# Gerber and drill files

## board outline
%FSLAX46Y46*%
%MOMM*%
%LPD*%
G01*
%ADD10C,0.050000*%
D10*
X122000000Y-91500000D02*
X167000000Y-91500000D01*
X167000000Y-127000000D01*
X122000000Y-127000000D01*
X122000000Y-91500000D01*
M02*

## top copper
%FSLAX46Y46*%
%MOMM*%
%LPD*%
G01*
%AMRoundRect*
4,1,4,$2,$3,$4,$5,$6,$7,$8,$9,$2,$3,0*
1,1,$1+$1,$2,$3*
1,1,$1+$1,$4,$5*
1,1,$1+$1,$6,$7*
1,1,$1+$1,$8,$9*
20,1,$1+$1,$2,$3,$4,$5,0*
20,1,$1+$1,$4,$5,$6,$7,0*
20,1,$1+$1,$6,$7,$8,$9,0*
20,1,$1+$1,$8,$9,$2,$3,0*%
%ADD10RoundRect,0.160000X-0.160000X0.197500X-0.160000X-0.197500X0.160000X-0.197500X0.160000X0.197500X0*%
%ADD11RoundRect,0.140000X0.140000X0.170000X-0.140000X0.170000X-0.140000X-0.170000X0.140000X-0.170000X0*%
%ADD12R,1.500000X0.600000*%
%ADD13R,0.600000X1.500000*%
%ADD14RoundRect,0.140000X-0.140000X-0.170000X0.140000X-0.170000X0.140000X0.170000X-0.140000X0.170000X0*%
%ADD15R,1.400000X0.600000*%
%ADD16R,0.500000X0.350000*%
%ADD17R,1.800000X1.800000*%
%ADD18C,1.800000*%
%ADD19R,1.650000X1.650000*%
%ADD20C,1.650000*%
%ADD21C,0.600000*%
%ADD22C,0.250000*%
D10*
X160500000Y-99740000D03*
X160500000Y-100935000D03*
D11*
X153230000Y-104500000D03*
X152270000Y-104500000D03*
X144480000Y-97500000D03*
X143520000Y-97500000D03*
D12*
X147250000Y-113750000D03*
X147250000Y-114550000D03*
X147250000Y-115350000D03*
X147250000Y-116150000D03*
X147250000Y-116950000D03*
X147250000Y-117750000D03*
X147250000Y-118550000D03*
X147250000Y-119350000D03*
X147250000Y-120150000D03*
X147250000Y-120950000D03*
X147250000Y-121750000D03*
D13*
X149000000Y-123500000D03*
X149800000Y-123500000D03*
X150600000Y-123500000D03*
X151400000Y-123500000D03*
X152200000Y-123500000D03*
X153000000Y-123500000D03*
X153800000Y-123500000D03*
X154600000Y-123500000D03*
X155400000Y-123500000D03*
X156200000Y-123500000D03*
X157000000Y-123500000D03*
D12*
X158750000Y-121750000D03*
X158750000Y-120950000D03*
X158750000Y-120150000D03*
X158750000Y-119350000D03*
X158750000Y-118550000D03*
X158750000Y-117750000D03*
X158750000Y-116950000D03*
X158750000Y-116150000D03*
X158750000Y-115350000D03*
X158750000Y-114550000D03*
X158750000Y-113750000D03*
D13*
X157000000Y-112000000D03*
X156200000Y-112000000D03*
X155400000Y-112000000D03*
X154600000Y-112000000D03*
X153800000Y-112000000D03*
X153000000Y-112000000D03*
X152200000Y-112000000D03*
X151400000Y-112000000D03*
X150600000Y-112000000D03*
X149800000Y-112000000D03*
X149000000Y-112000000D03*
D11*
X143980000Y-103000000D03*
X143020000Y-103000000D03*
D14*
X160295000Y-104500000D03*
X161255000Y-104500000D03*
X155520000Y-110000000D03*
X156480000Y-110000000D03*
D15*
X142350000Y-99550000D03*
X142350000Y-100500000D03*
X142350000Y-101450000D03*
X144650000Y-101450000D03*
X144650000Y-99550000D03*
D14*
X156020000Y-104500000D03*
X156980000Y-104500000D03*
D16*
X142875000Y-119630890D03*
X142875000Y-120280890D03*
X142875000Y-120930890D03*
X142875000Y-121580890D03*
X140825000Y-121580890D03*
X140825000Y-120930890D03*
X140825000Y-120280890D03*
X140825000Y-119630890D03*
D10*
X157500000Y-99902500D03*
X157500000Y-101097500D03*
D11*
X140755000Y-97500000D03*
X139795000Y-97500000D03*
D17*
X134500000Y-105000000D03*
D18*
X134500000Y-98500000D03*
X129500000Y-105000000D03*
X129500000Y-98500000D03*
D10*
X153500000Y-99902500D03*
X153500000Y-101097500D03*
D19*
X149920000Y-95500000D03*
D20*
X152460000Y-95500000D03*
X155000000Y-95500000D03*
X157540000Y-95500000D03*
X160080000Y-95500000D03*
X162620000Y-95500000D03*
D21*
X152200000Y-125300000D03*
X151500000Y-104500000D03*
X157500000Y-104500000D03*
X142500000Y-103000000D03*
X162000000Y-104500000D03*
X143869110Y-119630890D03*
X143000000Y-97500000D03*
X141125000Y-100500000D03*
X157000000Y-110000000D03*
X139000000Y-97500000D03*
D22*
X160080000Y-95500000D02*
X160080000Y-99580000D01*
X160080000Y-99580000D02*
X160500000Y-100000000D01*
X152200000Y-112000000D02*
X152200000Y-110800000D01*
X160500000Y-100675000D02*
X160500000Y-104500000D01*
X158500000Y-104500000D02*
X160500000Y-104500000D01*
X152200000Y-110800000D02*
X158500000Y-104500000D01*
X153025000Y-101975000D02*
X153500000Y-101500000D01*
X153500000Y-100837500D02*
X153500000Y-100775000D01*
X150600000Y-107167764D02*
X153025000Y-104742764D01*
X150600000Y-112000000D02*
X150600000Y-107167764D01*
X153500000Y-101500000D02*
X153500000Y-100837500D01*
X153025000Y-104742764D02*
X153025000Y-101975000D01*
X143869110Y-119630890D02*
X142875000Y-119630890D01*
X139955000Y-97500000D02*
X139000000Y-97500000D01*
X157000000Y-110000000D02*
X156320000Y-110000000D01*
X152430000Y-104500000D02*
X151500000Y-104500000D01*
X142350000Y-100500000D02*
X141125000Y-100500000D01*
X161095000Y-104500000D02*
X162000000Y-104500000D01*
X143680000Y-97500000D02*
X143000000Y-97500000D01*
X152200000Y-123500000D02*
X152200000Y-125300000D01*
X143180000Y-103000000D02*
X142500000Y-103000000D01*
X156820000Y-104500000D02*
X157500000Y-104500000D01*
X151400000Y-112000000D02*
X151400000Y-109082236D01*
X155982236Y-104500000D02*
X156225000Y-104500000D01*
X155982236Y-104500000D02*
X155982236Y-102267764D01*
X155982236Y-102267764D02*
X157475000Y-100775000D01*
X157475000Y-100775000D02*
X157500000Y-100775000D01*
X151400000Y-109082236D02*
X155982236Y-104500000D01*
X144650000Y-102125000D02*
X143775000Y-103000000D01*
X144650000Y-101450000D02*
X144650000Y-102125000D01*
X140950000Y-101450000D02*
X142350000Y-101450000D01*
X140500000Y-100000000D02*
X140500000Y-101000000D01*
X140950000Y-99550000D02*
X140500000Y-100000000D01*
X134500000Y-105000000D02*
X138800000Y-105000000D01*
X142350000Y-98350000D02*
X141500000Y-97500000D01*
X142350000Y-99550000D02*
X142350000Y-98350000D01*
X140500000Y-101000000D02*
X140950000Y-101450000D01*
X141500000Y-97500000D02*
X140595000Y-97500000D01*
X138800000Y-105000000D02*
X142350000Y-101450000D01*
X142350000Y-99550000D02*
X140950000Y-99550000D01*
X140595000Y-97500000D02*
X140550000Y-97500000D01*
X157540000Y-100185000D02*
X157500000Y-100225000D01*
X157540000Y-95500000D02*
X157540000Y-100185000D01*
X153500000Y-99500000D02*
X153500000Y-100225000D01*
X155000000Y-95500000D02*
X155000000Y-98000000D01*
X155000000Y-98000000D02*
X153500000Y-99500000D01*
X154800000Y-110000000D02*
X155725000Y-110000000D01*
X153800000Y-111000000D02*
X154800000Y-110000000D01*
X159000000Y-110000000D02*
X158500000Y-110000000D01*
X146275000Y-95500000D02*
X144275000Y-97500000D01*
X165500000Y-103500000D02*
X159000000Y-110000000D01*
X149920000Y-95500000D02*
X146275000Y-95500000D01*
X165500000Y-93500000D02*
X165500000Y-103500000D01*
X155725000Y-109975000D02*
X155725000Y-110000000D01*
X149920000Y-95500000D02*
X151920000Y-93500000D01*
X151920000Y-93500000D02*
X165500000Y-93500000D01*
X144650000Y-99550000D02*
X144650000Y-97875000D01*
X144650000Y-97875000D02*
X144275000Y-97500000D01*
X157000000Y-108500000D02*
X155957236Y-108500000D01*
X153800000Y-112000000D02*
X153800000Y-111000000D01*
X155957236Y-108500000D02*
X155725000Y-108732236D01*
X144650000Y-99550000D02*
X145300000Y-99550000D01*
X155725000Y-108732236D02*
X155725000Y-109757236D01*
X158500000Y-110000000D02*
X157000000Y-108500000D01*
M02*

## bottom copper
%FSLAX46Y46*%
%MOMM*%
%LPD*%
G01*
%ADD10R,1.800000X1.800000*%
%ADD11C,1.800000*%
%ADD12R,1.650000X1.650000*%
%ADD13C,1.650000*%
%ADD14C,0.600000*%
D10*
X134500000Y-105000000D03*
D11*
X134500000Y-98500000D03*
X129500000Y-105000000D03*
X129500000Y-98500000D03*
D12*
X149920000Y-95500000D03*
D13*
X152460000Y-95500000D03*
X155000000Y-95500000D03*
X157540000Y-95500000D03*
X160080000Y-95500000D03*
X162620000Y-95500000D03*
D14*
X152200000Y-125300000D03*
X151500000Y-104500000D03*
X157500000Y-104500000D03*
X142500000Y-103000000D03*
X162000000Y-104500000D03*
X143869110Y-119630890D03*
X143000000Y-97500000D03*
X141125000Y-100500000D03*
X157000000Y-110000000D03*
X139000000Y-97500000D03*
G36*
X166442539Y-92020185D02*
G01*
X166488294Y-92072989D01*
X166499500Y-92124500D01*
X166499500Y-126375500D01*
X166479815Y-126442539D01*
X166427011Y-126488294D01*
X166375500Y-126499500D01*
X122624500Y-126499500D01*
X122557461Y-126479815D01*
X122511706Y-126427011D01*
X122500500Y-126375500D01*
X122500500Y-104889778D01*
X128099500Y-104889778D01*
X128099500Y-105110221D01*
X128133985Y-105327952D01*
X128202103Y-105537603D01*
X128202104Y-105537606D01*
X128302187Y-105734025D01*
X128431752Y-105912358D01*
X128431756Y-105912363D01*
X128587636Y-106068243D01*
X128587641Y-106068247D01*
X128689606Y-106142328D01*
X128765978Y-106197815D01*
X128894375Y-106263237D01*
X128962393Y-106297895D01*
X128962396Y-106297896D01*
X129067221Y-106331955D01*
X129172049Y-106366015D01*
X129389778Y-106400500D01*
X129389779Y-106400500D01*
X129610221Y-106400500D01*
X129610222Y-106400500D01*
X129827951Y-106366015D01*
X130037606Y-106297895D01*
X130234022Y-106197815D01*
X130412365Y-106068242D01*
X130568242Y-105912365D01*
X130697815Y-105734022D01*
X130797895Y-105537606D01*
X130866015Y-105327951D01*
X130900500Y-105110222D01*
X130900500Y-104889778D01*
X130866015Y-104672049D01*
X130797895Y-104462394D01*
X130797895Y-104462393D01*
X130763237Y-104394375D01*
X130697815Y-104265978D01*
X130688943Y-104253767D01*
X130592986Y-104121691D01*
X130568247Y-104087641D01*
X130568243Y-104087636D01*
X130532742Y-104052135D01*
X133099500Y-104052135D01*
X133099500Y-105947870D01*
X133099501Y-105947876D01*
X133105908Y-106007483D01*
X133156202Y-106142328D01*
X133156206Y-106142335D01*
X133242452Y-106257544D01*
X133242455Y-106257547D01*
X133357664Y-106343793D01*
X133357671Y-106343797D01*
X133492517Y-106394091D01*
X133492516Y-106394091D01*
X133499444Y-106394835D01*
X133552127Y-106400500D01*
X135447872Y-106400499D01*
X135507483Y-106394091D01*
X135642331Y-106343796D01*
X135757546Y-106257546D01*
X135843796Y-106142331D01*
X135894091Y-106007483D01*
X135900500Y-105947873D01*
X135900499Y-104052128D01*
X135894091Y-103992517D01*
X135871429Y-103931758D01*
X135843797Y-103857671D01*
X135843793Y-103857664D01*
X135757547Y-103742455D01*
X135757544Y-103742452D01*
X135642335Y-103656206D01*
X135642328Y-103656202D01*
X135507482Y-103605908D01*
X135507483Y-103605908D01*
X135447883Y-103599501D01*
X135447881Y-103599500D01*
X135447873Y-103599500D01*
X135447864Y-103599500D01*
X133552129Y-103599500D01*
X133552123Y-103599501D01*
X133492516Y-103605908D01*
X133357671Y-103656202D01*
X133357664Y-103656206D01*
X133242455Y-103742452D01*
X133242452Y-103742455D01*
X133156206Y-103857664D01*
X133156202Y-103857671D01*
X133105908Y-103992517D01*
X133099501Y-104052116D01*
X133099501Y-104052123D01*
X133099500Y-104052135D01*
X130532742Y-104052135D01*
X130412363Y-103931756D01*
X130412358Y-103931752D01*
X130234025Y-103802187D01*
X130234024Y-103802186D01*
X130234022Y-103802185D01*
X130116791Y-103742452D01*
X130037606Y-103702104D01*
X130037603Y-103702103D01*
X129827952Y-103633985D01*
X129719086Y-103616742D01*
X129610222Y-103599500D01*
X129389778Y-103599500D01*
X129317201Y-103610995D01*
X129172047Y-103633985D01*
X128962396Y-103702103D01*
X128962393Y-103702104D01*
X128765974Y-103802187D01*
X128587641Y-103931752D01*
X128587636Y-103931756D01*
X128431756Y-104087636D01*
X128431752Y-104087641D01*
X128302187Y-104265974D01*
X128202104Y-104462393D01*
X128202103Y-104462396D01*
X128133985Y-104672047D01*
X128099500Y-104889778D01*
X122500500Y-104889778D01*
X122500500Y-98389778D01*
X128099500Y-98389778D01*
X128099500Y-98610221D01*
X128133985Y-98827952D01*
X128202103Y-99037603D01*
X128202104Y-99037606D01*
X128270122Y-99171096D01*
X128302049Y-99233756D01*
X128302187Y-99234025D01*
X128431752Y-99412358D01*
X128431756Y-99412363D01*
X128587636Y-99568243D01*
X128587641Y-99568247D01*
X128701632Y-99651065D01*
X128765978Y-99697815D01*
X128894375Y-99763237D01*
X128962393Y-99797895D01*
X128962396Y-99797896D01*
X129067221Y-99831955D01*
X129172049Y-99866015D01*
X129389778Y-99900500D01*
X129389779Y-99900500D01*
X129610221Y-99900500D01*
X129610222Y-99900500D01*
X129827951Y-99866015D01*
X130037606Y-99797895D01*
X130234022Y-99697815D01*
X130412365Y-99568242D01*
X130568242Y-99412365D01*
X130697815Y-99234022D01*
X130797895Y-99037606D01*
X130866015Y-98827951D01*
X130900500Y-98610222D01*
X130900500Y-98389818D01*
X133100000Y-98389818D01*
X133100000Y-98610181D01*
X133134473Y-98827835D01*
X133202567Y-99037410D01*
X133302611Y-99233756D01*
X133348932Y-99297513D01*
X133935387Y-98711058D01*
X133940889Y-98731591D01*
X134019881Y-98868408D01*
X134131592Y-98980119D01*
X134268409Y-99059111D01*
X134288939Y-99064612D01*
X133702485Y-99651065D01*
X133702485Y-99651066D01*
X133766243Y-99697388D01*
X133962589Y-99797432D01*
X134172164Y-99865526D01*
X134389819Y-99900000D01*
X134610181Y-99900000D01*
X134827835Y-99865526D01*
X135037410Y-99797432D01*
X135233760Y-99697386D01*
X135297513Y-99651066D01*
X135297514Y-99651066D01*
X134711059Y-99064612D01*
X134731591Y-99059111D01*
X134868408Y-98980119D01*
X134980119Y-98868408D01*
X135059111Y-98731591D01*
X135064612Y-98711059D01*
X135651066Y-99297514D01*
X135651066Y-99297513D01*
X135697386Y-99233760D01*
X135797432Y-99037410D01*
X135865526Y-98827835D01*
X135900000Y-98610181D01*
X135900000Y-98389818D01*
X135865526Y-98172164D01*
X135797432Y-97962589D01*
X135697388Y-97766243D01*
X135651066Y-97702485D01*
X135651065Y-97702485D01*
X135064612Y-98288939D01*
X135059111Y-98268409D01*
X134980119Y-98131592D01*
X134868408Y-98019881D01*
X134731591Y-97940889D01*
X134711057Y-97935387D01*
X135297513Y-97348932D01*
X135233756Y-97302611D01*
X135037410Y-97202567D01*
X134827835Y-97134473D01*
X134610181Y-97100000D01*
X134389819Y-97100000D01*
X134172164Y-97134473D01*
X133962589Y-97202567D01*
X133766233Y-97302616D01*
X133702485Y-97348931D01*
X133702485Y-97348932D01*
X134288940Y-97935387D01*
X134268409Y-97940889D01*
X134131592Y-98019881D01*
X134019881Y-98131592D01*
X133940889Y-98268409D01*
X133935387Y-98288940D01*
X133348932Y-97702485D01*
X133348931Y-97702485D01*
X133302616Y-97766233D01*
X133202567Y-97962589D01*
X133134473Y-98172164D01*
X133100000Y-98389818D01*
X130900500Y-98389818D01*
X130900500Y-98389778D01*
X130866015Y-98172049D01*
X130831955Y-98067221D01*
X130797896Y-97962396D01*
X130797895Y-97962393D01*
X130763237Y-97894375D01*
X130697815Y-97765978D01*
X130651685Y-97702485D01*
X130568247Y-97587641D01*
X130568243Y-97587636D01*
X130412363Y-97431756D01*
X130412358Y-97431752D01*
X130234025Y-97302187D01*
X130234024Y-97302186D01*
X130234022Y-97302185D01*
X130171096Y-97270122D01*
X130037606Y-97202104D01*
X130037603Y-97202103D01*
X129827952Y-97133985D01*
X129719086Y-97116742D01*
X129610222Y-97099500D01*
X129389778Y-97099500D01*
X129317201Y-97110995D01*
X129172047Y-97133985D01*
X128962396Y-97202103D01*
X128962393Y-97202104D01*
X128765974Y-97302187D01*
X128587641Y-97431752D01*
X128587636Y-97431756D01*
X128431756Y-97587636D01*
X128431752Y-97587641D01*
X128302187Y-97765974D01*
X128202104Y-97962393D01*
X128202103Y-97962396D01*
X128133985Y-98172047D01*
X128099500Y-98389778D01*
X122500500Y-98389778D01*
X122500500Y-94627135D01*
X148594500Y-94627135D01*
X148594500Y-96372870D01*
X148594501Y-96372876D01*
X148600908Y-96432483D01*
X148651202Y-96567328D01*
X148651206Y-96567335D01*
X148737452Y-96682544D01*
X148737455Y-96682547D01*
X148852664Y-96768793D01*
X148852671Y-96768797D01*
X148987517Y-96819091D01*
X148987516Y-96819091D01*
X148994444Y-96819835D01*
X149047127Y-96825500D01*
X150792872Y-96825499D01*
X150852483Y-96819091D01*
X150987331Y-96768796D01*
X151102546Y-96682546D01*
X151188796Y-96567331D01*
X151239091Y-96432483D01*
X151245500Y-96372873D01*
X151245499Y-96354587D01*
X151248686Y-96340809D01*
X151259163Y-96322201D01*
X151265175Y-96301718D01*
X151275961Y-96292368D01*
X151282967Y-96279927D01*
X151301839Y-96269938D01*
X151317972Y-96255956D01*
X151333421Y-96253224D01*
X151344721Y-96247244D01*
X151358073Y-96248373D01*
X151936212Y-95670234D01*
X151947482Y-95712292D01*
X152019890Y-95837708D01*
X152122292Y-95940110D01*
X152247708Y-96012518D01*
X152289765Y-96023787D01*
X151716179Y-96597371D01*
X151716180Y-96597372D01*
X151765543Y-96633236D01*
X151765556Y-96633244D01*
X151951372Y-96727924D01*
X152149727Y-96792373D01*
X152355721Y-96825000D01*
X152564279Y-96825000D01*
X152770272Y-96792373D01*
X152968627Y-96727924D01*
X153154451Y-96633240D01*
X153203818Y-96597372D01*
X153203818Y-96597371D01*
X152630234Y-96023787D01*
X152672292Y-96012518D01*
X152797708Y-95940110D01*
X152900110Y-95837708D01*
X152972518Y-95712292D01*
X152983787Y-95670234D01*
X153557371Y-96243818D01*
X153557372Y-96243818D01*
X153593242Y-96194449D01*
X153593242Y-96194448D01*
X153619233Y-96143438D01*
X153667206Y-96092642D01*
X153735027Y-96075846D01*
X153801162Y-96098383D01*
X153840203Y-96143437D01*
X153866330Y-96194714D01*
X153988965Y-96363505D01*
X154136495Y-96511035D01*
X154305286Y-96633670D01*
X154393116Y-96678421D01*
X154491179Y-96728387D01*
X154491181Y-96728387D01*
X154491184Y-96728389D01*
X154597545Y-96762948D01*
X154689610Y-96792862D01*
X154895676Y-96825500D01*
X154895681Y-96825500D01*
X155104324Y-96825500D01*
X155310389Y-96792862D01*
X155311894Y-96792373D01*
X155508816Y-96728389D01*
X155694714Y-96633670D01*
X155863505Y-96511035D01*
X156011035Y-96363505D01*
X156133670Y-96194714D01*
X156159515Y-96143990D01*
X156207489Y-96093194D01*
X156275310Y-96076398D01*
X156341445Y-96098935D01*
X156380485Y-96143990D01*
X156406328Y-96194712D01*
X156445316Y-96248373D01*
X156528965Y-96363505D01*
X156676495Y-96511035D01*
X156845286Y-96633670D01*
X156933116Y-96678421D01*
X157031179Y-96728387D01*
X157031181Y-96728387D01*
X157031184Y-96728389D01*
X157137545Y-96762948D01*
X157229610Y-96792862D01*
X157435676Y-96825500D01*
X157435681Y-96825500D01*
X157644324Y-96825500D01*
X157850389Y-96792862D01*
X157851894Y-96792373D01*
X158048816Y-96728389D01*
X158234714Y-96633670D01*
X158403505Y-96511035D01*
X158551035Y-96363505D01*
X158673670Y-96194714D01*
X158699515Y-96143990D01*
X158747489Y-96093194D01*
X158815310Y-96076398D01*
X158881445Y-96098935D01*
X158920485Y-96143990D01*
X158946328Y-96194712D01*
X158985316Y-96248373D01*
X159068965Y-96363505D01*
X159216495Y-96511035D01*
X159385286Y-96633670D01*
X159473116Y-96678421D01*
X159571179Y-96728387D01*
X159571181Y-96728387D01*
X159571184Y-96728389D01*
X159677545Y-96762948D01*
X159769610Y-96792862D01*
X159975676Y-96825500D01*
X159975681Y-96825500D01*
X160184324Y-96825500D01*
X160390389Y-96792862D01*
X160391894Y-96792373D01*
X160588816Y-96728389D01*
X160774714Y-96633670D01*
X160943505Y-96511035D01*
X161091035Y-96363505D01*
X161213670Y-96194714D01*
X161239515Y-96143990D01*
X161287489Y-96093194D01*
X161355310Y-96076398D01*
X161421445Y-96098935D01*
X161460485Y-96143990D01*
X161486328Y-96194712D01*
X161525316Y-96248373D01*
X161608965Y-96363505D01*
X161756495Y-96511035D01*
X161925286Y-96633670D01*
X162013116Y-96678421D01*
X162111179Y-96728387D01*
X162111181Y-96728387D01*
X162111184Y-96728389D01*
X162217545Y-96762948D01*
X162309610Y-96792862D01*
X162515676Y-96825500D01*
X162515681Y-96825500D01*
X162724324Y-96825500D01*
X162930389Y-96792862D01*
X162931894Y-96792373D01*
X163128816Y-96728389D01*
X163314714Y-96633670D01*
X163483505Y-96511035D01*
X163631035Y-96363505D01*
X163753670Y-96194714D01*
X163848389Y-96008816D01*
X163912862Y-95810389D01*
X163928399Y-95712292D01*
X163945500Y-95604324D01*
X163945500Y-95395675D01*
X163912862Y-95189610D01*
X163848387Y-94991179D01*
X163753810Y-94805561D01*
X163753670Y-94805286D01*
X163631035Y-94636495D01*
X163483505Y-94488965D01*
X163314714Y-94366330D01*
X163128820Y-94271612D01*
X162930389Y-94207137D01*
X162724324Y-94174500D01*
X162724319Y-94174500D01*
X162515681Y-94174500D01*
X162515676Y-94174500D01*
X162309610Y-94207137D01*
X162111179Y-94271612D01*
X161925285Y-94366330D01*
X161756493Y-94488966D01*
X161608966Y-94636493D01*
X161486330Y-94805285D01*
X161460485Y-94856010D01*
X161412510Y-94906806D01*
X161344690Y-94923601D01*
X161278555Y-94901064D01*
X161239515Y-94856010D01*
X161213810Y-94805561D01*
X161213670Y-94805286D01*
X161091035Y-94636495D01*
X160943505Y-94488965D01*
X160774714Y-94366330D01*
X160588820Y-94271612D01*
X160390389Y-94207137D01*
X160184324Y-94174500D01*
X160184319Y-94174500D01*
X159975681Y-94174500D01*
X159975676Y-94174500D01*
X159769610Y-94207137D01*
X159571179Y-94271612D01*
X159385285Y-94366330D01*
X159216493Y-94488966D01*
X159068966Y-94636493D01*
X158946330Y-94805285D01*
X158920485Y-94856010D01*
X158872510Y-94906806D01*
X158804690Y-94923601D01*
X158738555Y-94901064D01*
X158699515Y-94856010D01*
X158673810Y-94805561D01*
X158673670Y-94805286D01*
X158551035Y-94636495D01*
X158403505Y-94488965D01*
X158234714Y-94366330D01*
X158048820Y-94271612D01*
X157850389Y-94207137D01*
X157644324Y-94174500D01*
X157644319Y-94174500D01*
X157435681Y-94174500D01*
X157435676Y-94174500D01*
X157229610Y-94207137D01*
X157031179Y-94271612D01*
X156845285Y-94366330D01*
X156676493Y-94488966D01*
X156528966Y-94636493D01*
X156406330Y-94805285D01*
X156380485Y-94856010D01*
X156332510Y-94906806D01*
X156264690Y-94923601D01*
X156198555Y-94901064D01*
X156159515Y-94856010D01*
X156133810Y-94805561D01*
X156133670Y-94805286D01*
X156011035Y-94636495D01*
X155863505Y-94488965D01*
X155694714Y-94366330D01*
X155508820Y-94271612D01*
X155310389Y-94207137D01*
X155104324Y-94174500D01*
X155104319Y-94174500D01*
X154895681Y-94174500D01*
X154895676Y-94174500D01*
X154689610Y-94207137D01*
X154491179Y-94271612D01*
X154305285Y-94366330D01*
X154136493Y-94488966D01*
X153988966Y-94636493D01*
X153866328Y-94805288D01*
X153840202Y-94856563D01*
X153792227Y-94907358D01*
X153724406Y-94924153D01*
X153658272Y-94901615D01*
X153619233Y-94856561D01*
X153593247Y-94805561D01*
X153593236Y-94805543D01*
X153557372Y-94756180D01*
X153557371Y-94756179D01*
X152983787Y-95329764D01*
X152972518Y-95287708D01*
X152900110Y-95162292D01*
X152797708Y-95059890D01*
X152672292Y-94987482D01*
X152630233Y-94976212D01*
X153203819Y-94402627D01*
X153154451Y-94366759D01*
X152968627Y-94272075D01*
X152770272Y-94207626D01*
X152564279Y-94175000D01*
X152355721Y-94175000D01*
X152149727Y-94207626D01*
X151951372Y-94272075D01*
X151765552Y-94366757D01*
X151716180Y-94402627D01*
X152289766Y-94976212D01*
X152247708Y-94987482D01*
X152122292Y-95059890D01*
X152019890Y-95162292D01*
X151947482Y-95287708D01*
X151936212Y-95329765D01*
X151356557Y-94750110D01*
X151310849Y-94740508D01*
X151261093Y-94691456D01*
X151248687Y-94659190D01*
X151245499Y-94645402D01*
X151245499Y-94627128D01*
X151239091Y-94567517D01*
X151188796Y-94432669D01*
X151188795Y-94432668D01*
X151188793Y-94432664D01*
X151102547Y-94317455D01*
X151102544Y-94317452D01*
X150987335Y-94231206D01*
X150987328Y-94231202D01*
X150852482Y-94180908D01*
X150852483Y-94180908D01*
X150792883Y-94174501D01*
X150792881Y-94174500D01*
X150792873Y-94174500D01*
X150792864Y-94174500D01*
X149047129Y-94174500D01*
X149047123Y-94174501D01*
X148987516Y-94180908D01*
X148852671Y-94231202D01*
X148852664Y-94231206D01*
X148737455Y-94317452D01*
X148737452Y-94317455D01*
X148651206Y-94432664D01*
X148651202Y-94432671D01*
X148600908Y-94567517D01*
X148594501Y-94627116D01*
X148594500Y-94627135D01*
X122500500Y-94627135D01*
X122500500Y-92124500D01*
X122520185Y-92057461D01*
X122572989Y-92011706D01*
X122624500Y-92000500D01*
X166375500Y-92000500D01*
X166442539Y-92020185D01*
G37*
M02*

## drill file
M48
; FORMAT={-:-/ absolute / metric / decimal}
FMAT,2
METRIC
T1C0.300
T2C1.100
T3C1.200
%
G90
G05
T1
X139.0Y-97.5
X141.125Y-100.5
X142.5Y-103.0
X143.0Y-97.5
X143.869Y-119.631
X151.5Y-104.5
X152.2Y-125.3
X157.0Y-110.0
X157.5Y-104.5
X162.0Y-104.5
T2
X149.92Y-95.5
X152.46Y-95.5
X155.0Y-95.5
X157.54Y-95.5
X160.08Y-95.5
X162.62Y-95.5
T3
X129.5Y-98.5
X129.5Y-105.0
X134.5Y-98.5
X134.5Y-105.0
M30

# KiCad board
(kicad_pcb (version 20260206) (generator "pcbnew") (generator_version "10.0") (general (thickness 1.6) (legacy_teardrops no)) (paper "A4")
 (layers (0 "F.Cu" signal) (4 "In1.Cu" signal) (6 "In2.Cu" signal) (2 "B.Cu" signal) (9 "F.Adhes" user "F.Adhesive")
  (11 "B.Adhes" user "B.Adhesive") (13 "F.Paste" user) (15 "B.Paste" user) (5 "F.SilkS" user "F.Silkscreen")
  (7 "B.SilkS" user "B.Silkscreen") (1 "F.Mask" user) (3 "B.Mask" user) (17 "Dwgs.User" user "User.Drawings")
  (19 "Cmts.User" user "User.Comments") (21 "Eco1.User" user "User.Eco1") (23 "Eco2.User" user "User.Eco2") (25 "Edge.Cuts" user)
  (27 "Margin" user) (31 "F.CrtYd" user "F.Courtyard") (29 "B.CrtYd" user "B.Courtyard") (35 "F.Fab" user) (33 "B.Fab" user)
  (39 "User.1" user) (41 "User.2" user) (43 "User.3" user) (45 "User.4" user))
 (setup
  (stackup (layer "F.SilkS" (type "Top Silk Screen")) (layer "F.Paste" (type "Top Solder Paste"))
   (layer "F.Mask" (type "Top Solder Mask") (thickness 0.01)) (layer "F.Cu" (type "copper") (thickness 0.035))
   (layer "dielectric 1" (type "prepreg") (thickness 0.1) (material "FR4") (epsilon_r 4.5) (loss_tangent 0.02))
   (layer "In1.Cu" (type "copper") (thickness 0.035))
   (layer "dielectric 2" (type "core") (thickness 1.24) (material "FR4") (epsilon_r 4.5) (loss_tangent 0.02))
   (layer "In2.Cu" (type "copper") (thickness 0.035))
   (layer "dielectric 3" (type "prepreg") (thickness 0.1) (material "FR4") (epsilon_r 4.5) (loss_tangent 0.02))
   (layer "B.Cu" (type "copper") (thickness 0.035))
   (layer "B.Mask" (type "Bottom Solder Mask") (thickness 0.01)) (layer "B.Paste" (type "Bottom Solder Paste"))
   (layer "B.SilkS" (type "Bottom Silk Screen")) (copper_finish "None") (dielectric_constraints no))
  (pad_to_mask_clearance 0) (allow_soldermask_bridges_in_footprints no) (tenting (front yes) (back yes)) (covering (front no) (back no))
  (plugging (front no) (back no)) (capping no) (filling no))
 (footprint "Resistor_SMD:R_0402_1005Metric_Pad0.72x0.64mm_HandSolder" (layer "F.Cu") (at 160.5 100.3375 -90)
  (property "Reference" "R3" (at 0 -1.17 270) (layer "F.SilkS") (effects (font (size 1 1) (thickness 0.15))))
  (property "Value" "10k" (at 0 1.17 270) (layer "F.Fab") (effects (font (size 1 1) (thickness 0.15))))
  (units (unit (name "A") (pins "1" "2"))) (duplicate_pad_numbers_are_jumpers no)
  (pad "1" smd roundrect (at -0.5975 0 270) (size 0.715 0.64) (layers "F.Cu" "F.Mask" "F.Paste") (roundrect_rratio 0.25)
   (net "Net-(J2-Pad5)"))
  (pad "2" smd roundrect (at 0.5975 0 270) (size 0.715 0.64) (layers "F.Cu" "F.Mask" "F.Paste") (roundrect_rratio 0.25)
   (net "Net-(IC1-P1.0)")))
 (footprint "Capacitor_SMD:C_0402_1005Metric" (layer "F.Cu") (at 152.75 104.5 180)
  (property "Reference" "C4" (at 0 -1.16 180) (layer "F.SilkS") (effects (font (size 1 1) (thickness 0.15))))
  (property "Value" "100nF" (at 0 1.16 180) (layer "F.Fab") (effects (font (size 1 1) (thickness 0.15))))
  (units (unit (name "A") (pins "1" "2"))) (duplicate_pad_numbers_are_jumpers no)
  (pad "1" smd roundrect (at -0.48 0 180) (size 0.56 0.62) (layers "F.Cu" "F.Mask" "F.Paste") (roundrect_rratio 0.25) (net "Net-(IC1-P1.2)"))
  (pad "2" smd roundrect (at 0.48 0 180) (size 0.56 0.62) (layers "F.Cu" "F.Mask" "F.Paste") (roundrect_rratio 0.25) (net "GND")))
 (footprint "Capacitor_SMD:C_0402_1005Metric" (layer "F.Cu") (at 144 97.5 180)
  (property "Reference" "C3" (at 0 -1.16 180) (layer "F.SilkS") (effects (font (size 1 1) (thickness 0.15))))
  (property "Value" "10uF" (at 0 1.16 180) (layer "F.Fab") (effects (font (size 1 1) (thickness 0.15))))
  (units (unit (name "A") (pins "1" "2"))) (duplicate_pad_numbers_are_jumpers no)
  (pad "1" smd roundrect (at -0.48 0 180) (size 0.56 0.62) (layers "F.Cu" "F.Mask" "F.Paste") (roundrect_rratio 0.25)
   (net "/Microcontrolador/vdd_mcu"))
  (pad "2" smd roundrect (at 0.48 0 180) (size 0.56 0.62) (layers "F.Cu" "F.Mask" "F.Paste") (roundrect_rratio 0.25) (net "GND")))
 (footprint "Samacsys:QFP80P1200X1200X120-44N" (layer "F.Cu") (at 153 117.75)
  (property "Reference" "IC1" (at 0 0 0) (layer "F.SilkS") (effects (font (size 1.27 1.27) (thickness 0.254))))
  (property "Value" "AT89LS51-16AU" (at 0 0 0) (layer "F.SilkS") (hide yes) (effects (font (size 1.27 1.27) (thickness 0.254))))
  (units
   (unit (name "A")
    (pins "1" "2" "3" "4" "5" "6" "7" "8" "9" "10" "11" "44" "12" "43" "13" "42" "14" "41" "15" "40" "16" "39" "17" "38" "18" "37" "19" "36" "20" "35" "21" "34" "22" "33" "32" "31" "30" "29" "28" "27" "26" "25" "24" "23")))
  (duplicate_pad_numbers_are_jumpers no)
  (pad "1" smd rect (at -5.75 -4 90) (size 0.6 1.5) (layers "F.Cu" "F.Mask" "F.Paste") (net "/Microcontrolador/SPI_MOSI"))
  (pad "2" smd rect (at -5.75 -3.2 90) (size 0.6 1.5) (layers "F.Cu" "F.Mask" "F.Paste") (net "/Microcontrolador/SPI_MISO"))
  (pad "3" smd rect (at -5.75 -2.4 90) (size 0.6 1.5) (layers "F.Cu" "F.Mask" "F.Paste") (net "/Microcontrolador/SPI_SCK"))
  (pad "4" smd rect (at -5.75 -1.6 90) (size 0.6 1.5) (layers "F.Cu" "F.Mask" "F.Paste") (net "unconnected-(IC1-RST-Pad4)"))
  (pad "5" smd rect (at -5.75 -0.8 90) (size 0.6 1.5) (layers "F.Cu" "F.Mask" "F.Paste") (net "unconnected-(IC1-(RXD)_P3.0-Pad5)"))
  (pad "6" smd rect (at -5.75 0 90) (size 0.6 1.5) (layers "F.Cu" "F.Mask" "F.Paste") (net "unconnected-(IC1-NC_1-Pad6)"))
  (pad "7" smd rect (at -5.75 0.8 90) (size 0.6 1.5) (layers "F.Cu" "F.Mask" "F.Paste") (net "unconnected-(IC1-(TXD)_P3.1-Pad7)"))
  (pad "8" smd rect (at -5.75 1.6 90) (size 0.6 1.5) (layers "F.Cu" "F.Mask" "F.Paste") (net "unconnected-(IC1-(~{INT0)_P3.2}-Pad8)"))
  (pad "9" smd rect (at -5.75 2.4 90) (size 0.6 1.5) (layers "F.Cu" "F.Mask" "F.Paste") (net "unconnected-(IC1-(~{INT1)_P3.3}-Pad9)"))
  (pad "10" smd rect (at -5.75 3.2 90) (size 0.6 1.5) (layers "F.Cu" "F.Mask" "F.Paste") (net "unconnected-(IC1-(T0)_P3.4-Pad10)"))
  (pad "11" smd rect (at -5.75 4 90) (size 0.6 1.5) (layers "F.Cu" "F.Mask" "F.Paste") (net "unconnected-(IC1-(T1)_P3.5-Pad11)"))
  (pad "12" smd rect (at -4 5.75) (size 0.6 1.5) (layers "F.Cu" "F.Mask" "F.Paste") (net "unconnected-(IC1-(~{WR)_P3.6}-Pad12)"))
  (pad "13" smd rect (at -3.2 5.75) (size 0.6 1.5) (layers "F.Cu" "F.Mask" "F.Paste") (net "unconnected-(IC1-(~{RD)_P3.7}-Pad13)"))
  (pad "14" smd rect (at -2.4 5.75) (size 0.6 1.5) (layers "F.Cu" "F.Mask" "F.Paste") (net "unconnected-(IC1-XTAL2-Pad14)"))
  (pad "15" smd rect (at -1.6 5.75) (size 0.6 1.5) (layers "F.Cu" "F.Mask" "F.Paste") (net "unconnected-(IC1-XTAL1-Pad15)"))
  (pad "16" smd rect (at -0.8 5.75) (size 0.6 1.5) (layers "F.Cu" "F.Mask" "F.Paste") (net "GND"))
  (pad "17" smd rect (at 0 5.75) (size 0.6 1.5) (layers "F.Cu" "F.Mask" "F.Paste") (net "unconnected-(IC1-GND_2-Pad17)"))
  (pad "18" smd rect (at 0.8 5.75) (size 0.6 1.5) (layers "F.Cu" "F.Mask" "F.Paste") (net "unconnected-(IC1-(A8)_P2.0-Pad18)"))
  (pad "19" smd rect (at 1.6 5.75) (size 0.6 1.5) (layers "F.Cu" "F.Mask" "F.Paste") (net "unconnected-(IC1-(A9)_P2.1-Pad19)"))
  (pad "20" smd rect (at 2.4 5.75) (size 0.6 1.5) (layers "F.Cu" "F.Mask" "F.Paste") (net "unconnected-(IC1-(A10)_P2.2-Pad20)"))
  (pad "21" smd rect (at 3.2 5.75) (size 0.6 1.5) (layers "F.Cu" "F.Mask" "F.Paste") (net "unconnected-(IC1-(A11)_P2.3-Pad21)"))
  (pad "22" smd rect (at 4 5.75) (size 0.6 1.5) (layers "F.Cu" "F.Mask" "F.Paste") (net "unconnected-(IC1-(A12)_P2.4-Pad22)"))
  (pad "23" smd rect (at 5.75 4 90) (size 0.6 1.5) (layers "F.Cu" "F.Mask" "F.Paste") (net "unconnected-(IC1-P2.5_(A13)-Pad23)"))
  (pad "24" smd rect (at 5.75 3.2 90) (size 0.6 1.5) (layers "F.Cu" "F.Mask" "F.Paste") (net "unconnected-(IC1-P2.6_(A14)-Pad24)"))
  (pad "25" smd rect (at 5.75 2.4 90) (size 0.6 1.5) (layers "F.Cu" "F.Mask" "F.Paste") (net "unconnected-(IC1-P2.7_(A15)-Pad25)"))
  (pad "26" smd rect (at 5.75 1.6 90) (size 0.6 1.5) (layers "F.Cu" "F.Mask" "F.Paste") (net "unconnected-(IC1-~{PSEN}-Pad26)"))
  (pad "27" smd rect (at 5.75 0.8 90) (size 0.6 1.5) (layers "F.Cu" "F.Mask" "F.Paste") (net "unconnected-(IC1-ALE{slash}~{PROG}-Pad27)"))
  (pad "28" smd rect (at 5.75 0 90) (size 0.6 1.5) (layers "F.Cu" "F.Mask" "F.Paste") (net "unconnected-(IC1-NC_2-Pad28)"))
  (pad "29" smd rect (at 5.75 -0.8 90) (size 0.6 1.5) (layers "F.Cu" "F.Mask" "F.Paste") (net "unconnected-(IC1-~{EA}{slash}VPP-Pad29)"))
  (pad "30" smd rect (at 5.75 -1.6 90) (size 0.6 1.5) (layers "F.Cu" "F.Mask" "F.Paste") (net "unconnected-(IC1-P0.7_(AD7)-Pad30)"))
  (pad "31" smd rect (at 5.75 -2.4 90) (size 0.6 1.5) (layers "F.Cu" "F.Mask" "F.Paste") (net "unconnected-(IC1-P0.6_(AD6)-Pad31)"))
  (pad "32" smd rect (at 5.75 -3.2 90) (size 0.6 1.5) (layers "F.Cu" "F.Mask" "F.Paste") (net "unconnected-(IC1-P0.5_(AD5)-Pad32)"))
  (pad "33" smd rect (at 5.75 -4 90) (size 0.6 1.5) (layers "F.Cu" "F.Mask" "F.Paste") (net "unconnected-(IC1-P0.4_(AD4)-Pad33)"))
  (pad "34" smd rect (at 4 -5.75) (size 0.6 1.5) (layers "F.Cu" "F.Mask" "F.Paste") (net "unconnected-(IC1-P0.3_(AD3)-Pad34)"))
  (pad "35" smd rect (at 3.2 -5.75) (size 0.6 1.5) (layers "F.Cu" "F.Mask" "F.Paste") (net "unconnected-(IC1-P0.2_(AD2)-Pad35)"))
  (pad "36" smd rect (at 2.4 -5.75) (size 0.6 1.5) (layers "F.Cu" "F.Mask" "F.Paste") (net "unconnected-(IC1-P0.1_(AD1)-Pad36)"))
  (pad "37" smd rect (at 1.6 -5.75) (size 0.6 1.5) (layers "F.Cu" "F.Mask" "F.Paste") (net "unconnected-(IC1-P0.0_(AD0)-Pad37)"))
  (pad "38" smd rect (at 0.8 -5.75) (size 0.6 1.5) (layers "F.Cu" "F.Mask" "F.Paste") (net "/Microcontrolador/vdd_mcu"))
  (pad "39" smd rect (at 0 -5.75) (size 0.6 1.5) (layers "F.Cu" "F.Mask" "F.Paste") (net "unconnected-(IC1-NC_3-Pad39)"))
  (pad "40" smd rect (at -0.8 -5.75) (size 0.6 1.5) (layers "F.Cu" "F.Mask" "F.Paste") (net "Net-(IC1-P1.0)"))
  (pad "41" smd rect (at -1.6 -5.75) (size 0.6 1.5) (layers "F.Cu" "F.Mask" "F.Paste") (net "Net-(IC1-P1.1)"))
  (pad "42" smd rect (at -2.4 -5.75) (size 0.6 1.5) (layers "F.Cu" "F.Mask" "F.Paste") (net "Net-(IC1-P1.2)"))
  (pad "43" smd rect (at -3.2 -5.75) (size 0.6 1.5) (layers "F.Cu" "F.Mask" "F.Paste") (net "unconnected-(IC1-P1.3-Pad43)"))
  (pad "44" smd rect (at -4 -5.75) (size 0.6 1.5) (layers "F.Cu" "F.Mask" "F.Paste") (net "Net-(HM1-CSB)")))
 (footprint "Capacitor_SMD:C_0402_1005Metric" (layer "F.Cu") (at 143.5 103 180)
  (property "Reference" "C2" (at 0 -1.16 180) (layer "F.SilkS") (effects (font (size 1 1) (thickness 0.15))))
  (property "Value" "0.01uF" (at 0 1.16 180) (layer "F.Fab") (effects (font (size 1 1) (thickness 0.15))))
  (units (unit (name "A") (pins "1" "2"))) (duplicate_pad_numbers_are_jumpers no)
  (pad "1" smd roundrect (at -0.48 0 180) (size 0.56 0.62) (layers "F.Cu" "F.Mask" "F.Paste") (roundrect_rratio 0.25)
   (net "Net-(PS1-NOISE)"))
  (pad "2" smd roundrect (at 0.48 0 180) (size 0.56 0.62) (layers "F.Cu" "F.Mask" "F.Paste") (roundrect_rratio 0.25) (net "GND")))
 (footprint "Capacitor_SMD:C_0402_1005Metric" (layer "F.Cu") (at 160.775 104.5)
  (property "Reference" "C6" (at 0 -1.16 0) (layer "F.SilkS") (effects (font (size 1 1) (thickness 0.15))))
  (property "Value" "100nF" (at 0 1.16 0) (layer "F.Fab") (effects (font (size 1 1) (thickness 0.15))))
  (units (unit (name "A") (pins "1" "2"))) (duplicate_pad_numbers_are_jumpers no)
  (pad "1" smd roundrect (at -0.48 0) (size 0.56 0.62) (layers "F.Cu" "F.Mask" "F.Paste") (roundrect_rratio 0.25) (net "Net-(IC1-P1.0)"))
  (pad "2" smd roundrect (at 0.48 0) (size 0.56 0.62) (layers "F.Cu" "F.Mask" "F.Paste") (roundrect_rratio 0.25) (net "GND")))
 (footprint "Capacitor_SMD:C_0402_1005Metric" (layer "F.Cu") (at 156 110)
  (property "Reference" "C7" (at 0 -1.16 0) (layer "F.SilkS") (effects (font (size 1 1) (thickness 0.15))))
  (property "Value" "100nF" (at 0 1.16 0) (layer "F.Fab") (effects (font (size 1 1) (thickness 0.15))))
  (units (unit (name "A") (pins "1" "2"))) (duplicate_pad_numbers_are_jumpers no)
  (pad "1" smd roundrect (at -0.48 0) (size 0.56 0.62) (layers "F.Cu" "F.Mask" "F.Paste") (roundrect_rratio 0.25)
   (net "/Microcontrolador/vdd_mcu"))
  (pad "2" smd roundrect (at 0.48 0) (size 0.56 0.62) (layers "F.Cu" "F.Mask" "F.Paste") (roundrect_rratio 0.25) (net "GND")))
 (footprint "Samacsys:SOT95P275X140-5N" (layer "F.Cu") (at 143.5 100.5)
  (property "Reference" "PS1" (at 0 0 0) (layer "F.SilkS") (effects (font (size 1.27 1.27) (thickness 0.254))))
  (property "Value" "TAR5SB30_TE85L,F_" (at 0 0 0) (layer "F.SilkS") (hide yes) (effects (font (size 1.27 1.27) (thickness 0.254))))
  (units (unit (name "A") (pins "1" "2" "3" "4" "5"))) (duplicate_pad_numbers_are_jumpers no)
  (pad "1" smd rect (at -1.15 -0.95 90) (size 0.6 1.4) (layers "F.Cu" "F.Mask" "F.Paste") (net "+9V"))
  (pad "2" smd rect (at -1.15 0 90) (size 0.6 1.4) (layers "F.Cu" "F.Mask" "F.Paste") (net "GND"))
  (pad "3" smd rect (at -1.15 0.95 90) (size 0.6 1.4) (layers "F.Cu" "F.Mask" "F.Paste") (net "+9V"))
  (pad "4" smd rect (at 1.15 0.95 90) (size 0.6 1.4) (layers "F.Cu" "F.Mask" "F.Paste") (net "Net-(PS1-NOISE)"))
  (pad "5" smd rect (at 1.15 -0.95 90) (size 0.6 1.4) (layers "F.Cu" "F.Mask" "F.Paste") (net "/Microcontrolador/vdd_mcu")))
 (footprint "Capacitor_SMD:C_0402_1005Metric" (layer "F.Cu") (at 156.5 104.5)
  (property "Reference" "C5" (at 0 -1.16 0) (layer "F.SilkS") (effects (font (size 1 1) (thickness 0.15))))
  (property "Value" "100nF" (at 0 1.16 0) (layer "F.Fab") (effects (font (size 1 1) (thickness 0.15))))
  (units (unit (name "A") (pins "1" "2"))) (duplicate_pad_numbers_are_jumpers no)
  (pad "1" smd roundrect (at -0.48 0) (size 0.56 0.62) (layers "F.Cu" "F.Mask" "F.Paste") (roundrect_rratio 0.25) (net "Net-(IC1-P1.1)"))
  (pad "2" smd roundrect (at 0.48 0) (size 0.56 0.62) (layers "F.Cu" "F.Mask" "F.Paste") (roundrect_rratio 0.25) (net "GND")))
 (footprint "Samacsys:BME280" (layer "F.Cu") (at 140.825 119.63089)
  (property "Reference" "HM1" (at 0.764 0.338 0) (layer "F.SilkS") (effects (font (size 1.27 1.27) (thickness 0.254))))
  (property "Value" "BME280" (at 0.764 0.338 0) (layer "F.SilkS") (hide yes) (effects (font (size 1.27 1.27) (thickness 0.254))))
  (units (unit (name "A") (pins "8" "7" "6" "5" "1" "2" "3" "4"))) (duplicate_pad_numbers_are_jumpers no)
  (pad "1" smd rect (at 2.05 0 90) (size 0.35 0.5) (layers "F.Cu" "F.Mask" "F.Paste") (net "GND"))
  (pad "2" smd rect (at 2.05 0.65 90) (size 0.35 0.5) (layers "F.Cu" "F.Mask" "F.Paste") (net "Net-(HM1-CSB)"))
  (pad "3" smd rect (at 2.05 1.3 90) (size 0.35 0.5) (layers "F.Cu" "F.Mask" "F.Paste") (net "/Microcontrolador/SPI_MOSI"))
  (pad "4" smd rect (at 2.05 1.95 90) (size 0.35 0.5) (layers "F.Cu" "F.Mask" "F.Paste") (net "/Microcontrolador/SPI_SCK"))
  (pad "5" smd rect (at 0 1.95 90) (size 0.35 0.5) (layers "F.Cu" "F.Mask" "F.Paste") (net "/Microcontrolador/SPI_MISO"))
  (pad "6" smd rect (at 0 1.3 90) (size 0.35 0.5) (layers "F.Cu" "F.Mask" "F.Paste") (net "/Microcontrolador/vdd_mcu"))
  (pad "7" smd rect (at 0 0.65 90) (size 0.35 0.5) (layers "F.Cu" "F.Mask" "F.Paste") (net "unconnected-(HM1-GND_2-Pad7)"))
  (pad "8" smd rect (at 0 0 90) (size 0.35 0.5) (layers "F.Cu" "F.Mask" "F.Paste") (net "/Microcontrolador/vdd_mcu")))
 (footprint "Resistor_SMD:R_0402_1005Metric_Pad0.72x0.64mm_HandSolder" (layer "F.Cu") (at 157.5 100.5 -90)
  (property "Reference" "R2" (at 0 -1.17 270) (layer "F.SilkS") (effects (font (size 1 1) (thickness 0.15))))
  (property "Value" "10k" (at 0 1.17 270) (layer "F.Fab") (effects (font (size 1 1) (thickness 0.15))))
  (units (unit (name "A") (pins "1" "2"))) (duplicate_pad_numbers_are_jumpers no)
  (pad "1" smd roundrect (at -0.5975 0 270) (size 0.715 0.64) (layers "F.Cu" "F.Mask" "F.Paste") (roundrect_rratio 0.25)
   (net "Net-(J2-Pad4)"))
  (pad "2" smd roundrect (at 0.5975 0 270) (size 0.715 0.64) (layers "F.Cu" "F.Mask" "F.Paste") (roundrect_rratio 0.25)
   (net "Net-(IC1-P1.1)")))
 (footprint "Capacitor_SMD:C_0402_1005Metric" (layer "F.Cu") (at 140.275 97.5 180)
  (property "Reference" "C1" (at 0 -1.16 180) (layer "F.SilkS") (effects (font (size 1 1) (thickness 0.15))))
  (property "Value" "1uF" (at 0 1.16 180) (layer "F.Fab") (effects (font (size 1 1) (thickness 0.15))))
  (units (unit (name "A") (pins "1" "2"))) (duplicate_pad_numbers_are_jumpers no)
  (pad "1" smd roundrect (at -0.48 0 180) (size 0.56 0.62) (layers "F.Cu" "F.Mask" "F.Paste") (roundrect_rratio 0.25) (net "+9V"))
  (pad "2" smd roundrect (at 0.48 0 180) (size 0.56 0.62) (layers "F.Cu" "F.Mask" "F.Paste") (roundrect_rratio 0.25) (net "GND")))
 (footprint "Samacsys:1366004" (layer "F.Cu") (at 134.5 105 180)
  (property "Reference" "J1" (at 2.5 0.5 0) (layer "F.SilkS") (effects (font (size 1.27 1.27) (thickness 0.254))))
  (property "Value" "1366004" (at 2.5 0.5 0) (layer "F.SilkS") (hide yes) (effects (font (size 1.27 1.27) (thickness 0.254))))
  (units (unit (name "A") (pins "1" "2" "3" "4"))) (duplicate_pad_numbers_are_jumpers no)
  (pad "1" thru_hole rect (at 0 0 180) (size 1.8 1.8) (drill 1.2) (layers "*.Cu" "*.Mask") (remove_unused_layers no) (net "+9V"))
  (pad "2" thru_hole circle (at 0 6.5 180) (size 1.8 1.8) (drill 1.2) (layers "*.Cu" "*.Mask") (remove_unused_layers no) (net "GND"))
  (pad "3" thru_hole circle (at 5 0 180) (size 1.8 1.8) (drill 1.2) (layers "*.Cu" "*.Mask") (remove_unused_layers no)
   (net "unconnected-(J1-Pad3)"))
  (pad "4" thru_hole circle (at 5 6.5 180) (size 1.8 1.8) (drill 1.2) (layers "*.Cu" "*.Mask") (remove_unused_layers no)
   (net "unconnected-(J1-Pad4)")))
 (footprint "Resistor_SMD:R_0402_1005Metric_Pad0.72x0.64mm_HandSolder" (layer "F.Cu") (at 153.5 100.5 -90)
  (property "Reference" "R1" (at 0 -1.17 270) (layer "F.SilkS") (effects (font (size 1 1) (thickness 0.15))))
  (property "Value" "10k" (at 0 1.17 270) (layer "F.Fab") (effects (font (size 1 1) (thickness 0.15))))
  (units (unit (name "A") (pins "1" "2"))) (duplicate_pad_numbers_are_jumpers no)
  (pad "1" smd roundrect (at -0.5975 0 270) (size 0.715 0.64) (layers "F.Cu" "F.Mask" "F.Paste") (roundrect_rratio 0.25)
   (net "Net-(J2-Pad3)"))
  (pad "2" smd roundrect (at 0.5975 0 270) (size 0.715 0.64) (layers "F.Cu" "F.Mask" "F.Paste") (roundrect_rratio 0.25)
   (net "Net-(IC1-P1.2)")))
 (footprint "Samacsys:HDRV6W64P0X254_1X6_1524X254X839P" (layer "F.Cu") (at 149.92 95.5)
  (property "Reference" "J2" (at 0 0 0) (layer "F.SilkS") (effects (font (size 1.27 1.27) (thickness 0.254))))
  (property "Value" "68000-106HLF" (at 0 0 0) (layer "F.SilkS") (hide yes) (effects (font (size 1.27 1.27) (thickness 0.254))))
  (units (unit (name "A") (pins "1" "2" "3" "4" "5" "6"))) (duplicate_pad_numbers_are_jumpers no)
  (pad "1" thru_hole rect (at 0 0) (size 1.65 1.65) (drill 1.1) (layers "*.Cu" "*.Mask") (remove_unused_layers no)
   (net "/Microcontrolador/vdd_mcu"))
  (pad "2" thru_hole circle (at 2.54 0) (size 1.65 1.65) (drill 1.1) (layers "*.Cu" "*.Mask") (remove_unused_layers no) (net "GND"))
  (pad "3" thru_hole circle (at 5.08 0) (size 1.65 1.65) (drill 1.1) (layers "*.Cu" "*.Mask") (remove_unused_layers no)
   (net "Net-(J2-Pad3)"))
  (pad "4" thru_hole circle (at 7.62 0) (size 1.65 1.65) (drill 1.1) (layers "*.Cu" "*.Mask") (remove_unused_layers no)
   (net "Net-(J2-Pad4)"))
  (pad "5" thru_hole circle (at 10.16 0) (size 1.65 1.65) (drill 1.1) (layers "*.Cu" "*.Mask") (remove_unused_layers no)
   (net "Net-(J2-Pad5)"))
  (pad "6" thru_hole circle (at 12.7 0) (size 1.65 1.65) (drill 1.1) (layers "*.Cu" "*.Mask") (remove_unused_layers no)
   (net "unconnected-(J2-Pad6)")))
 (gr_rect (start 122 91.5) (end 167 127) (stroke (width 0.05) (type default)) (fill no) (layer "Edge.Cuts"))
 (segment (start 160.08 95.5) (end 160.08 99.58) (width 0.25) (layer "F.Cu") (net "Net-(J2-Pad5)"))
 (segment (start 160.08 99.58) (end 160.5 100) (width 0.25) (layer "F.Cu") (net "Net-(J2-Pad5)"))
 (segment (start 152.2 112) (end 152.2 110.8) (width 0.25) (layer "F.Cu") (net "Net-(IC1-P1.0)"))
 (segment (start 160.5 100.675) (end 160.5 104.5) (width 0.25) (layer "F.Cu") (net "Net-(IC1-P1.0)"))
 (segment (start 158.5 104.5) (end 160.5 104.5) (width 0.25) (layer "F.Cu") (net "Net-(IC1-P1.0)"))
 (segment (start 152.2 110.8) (end 158.5 104.5) (width 0.25) (layer "F.Cu") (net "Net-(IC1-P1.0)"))
 (segment (start 153.025 101.975) (end 153.5 101.5) (width 0.25) (layer "F.Cu") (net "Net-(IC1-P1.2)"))
 (segment (start 153.5 100.8375) (end 153.5 100.775) (width 0.25) (layer "F.Cu") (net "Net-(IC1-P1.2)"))
 (segment (start 150.6 107.167764) (end 153.025 104.742764) (width 0.25) (layer "F.Cu") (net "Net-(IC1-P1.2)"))
 (segment (start 150.6 112) (end 150.6 107.167764) (width 0.25) (layer "F.Cu") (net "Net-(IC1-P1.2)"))
 (segment (start 153.5 101.5) (end 153.5 100.8375) (width 0.25) (layer "F.Cu") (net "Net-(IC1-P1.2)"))
 (segment (start 153.025 104.742764) (end 153.025 101.975) (width 0.25) (layer "F.Cu") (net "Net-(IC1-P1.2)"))
 (segment (start 143.86911 119.63089) (end 142.875 119.63089) (width 0.25) (layer "F.Cu") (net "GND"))
 (segment (start 139.955 97.5) (end 139 97.5) (width 0.25) (layer "F.Cu") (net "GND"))
 (segment (start 157 110) (end 156.32 110) (width 0.25) (layer "F.Cu") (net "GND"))
 (segment (start 152.43 104.5) (end 151.5 104.5) (width 0.25) (layer "F.Cu") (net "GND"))
 (segment (start 142.35 100.5) (end 141.125 100.5) (width 0.25) (layer "F.Cu") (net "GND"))
 (segment (start 161.095 104.5) (end 162 104.5) (width 0.25) (layer "F.Cu") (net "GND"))
 (segment (start 143.68 97.5) (end 143 97.5) (width 0.25) (layer "F.Cu") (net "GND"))
 (segment (start 152.2 123.5) (end 152.2 125.3) (width 0.25) (layer "F.Cu") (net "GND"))
 (segment (start 143.18 103) (end 142.5 103) (width 0.25) (layer "F.Cu") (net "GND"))
 (segment (start 156.82 104.5) (end 157.5 104.5) (width 0.25) (layer "F.Cu") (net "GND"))
 (via (at 152.2 125.3) (size 0.6) (drill 0.3) (layers "F.Cu" "B.Cu") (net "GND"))
 (via (at 151.5 104.5) (size 0.6) (drill 0.3) (layers "F.Cu" "B.Cu") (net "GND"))
 (via (at 157.5 104.5) (size 0.6) (drill 0.3) (layers "F.Cu" "B.Cu") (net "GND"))
 (via (at 142.5 103) (size 0.6) (drill 0.3) (layers "F.Cu" "B.Cu") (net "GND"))
 (via (at 162 104.5) (size 0.6) (drill 0.3) (layers "F.Cu" "B.Cu") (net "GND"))
 (via (at 143.86911 119.63089) (size 0.6) (drill 0.3) (layers "F.Cu" "B.Cu") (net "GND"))
 (via (at 143 97.5) (size 0.6) (drill 0.3) (layers "F.Cu" "B.Cu") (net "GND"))
 (via (at 141.125 100.5) (size 0.6) (drill 0.3) (layers "F.Cu" "B.Cu") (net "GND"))
 (via (at 157 110) (size 0.6) (drill 0.3) (layers "F.Cu" "B.Cu") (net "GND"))
 (via (at 139 97.5) (size 0.6) (drill 0.3) (layers "F.Cu" "B.Cu") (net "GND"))
 (segment (start 151.4 112) (end 151.4 109.082236) (width 0.25) (layer "F.Cu") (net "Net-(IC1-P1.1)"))
 (segment (start 155.982236 104.5) (end 156.225 104.5) (width 0.25) (layer "F.Cu") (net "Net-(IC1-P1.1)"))
 (segment (start 155.982236 104.5) (end 155.982236 102.267764) (width 0.25) (layer "F.Cu") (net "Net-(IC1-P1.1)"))
 (segment (start 155.982236 102.267764) (end 157.475 100.775) (width 0.25) (layer "F.Cu") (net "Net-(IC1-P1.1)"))
 (segment (start 157.475 100.775) (end 157.5 100.775) (width 0.25) (layer "F.Cu") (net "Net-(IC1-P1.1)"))
 (segment (start 151.4 109.082236) (end 155.982236 104.5) (width 0.25) (layer "F.Cu") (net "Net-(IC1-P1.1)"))
 (segment (start 144.65 102.125) (end 143.775 103) (width 0.25) (layer "F.Cu") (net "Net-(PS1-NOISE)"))
 (segment (start 144.65 101.45) (end 144.65 102.125) (width 0.25) (layer "F.Cu") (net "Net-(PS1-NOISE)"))
 (segment (start 140.95 101.45) (end 142.35 101.45) (width 0.25) (layer "F.Cu") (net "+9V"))
 (segment (start 140.5 100) (end 140.5 101) (width 0.25) (layer "F.Cu") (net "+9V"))
 (segment (start 140.95 99.55) (end 140.5 100) (width 0.25) (layer "F.Cu") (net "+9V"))
 (segment (start 134.5 105) (end 138.8 105) (width 0.25) (layer "F.Cu") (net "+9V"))
 (segment (start 142.35 98.35) (end 141.5 97.5) (width 0.25) (layer "F.Cu") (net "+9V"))
 (segment (start 142.35 99.55) (end 142.35 98.35) (width 0.25) (layer "F.Cu") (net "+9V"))
 (segment (start 140.5 101) (end 140.95 101.45) (width 0.25) (layer "F.Cu") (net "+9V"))
 (segment (start 141.5 97.5) (end 140.595 97.5) (width 0.25) (layer "F.Cu") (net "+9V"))
 (segment (start 138.8 105) (end 142.35 101.45) (width 0.25) (layer "F.Cu") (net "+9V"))
 (segment (start 142.35 99.55) (end 140.95 99.55) (width 0.25) (layer "F.Cu") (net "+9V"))
 (segment (start 140.595 97.5) (end 140.55 97.5) (width 0.25) (layer "F.Cu") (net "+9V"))
 (segment (start 157.54 100.185) (end 157.5 100.225) (width 0.25) (layer "F.Cu") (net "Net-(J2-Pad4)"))
 (segment (start 157.54 95.5) (end 157.54 100.185) (width 0.25) (layer "F.Cu") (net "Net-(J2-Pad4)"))
 (segment (start 153.5 99.5) (end 153.5 100.225) (width 0.25) (layer "F.Cu") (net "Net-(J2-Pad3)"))
 (segment (start 155 95.5) (end 155 98) (width 0.25) (layer "F.Cu") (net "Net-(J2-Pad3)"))
 (segment (start 155 98) (end 153.5 99.5) (width 0.25) (layer "F.Cu") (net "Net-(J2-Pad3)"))
 (segment (start 154.8 110) (end 155.725 110) (width 0.25) (layer "F.Cu") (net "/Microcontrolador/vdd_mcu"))
 (segment (start 153.8 111) (end 154.8 110) (width 0.25) (layer "F.Cu") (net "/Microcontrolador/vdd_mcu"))
 (segment (start 159 110) (end 158.5 110) (width 0.25) (layer "F.Cu") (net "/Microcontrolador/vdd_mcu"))
 (segment (start 146.275 95.5) (end 144.275 97.5) (width 0.25) (layer "F.Cu") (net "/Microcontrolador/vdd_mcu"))
 (segment (start 165.5 103.5) (end 159 110) (width 0.25) (layer "F.Cu") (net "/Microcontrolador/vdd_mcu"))
 (segment (start 149.92 95.5) (end 146.275 95.5) (width 0.25) (layer "F.Cu") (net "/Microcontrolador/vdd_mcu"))
 (segment (start 165.5 93.5) (end 165.5 103.5) (width 0.25) (layer "F.Cu") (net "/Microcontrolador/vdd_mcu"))
 (segment (start 155.725 109.975) (end 155.725 110) (width 0.25) (layer "F.Cu") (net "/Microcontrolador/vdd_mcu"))
 (segment (start 149.92 95.5) (end 151.92 93.5) (width 0.25) (layer "F.Cu") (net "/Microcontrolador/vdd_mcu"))
 (segment (start 151.92 93.5) (end 165.5 93.5) (width 0.25) (layer "F.Cu") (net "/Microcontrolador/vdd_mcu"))
 (segment (start 144.65 99.55) (end 144.65 97.875) (width 0.25) (layer "F.Cu") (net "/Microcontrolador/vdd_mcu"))
 (segment (start 144.65 97.875) (end 144.275 97.5) (width 0.25) (layer "F.Cu") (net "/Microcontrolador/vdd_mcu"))
 (segment (start 157 108.5) (end 155.957236 108.5) (width 0.25) (layer "F.Cu") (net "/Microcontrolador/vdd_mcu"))
 (segment (start 153.8 112) (end 153.8 111) (width 0.25) (layer "F.Cu") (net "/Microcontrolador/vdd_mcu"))
 (segment (start 155.957236 108.5) (end 155.725 108.732236) (width 0.25) (layer "F.Cu") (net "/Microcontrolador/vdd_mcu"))
 (segment (start 144.65 99.55) (end 145.3 99.55) (width 0.25) (layer "F.Cu") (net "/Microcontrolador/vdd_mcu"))
 (segment (start 155.725 108.732236) (end 155.725 109.757236) (width 0.25) (layer "F.Cu") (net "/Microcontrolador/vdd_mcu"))
 (segment (start 158.5 110) (end 157 108.5) (width 0.25) (layer "F.Cu") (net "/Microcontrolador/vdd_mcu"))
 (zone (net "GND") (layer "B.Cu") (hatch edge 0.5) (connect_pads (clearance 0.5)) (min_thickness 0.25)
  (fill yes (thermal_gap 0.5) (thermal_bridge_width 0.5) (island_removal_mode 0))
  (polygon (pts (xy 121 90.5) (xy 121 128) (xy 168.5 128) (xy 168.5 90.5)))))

